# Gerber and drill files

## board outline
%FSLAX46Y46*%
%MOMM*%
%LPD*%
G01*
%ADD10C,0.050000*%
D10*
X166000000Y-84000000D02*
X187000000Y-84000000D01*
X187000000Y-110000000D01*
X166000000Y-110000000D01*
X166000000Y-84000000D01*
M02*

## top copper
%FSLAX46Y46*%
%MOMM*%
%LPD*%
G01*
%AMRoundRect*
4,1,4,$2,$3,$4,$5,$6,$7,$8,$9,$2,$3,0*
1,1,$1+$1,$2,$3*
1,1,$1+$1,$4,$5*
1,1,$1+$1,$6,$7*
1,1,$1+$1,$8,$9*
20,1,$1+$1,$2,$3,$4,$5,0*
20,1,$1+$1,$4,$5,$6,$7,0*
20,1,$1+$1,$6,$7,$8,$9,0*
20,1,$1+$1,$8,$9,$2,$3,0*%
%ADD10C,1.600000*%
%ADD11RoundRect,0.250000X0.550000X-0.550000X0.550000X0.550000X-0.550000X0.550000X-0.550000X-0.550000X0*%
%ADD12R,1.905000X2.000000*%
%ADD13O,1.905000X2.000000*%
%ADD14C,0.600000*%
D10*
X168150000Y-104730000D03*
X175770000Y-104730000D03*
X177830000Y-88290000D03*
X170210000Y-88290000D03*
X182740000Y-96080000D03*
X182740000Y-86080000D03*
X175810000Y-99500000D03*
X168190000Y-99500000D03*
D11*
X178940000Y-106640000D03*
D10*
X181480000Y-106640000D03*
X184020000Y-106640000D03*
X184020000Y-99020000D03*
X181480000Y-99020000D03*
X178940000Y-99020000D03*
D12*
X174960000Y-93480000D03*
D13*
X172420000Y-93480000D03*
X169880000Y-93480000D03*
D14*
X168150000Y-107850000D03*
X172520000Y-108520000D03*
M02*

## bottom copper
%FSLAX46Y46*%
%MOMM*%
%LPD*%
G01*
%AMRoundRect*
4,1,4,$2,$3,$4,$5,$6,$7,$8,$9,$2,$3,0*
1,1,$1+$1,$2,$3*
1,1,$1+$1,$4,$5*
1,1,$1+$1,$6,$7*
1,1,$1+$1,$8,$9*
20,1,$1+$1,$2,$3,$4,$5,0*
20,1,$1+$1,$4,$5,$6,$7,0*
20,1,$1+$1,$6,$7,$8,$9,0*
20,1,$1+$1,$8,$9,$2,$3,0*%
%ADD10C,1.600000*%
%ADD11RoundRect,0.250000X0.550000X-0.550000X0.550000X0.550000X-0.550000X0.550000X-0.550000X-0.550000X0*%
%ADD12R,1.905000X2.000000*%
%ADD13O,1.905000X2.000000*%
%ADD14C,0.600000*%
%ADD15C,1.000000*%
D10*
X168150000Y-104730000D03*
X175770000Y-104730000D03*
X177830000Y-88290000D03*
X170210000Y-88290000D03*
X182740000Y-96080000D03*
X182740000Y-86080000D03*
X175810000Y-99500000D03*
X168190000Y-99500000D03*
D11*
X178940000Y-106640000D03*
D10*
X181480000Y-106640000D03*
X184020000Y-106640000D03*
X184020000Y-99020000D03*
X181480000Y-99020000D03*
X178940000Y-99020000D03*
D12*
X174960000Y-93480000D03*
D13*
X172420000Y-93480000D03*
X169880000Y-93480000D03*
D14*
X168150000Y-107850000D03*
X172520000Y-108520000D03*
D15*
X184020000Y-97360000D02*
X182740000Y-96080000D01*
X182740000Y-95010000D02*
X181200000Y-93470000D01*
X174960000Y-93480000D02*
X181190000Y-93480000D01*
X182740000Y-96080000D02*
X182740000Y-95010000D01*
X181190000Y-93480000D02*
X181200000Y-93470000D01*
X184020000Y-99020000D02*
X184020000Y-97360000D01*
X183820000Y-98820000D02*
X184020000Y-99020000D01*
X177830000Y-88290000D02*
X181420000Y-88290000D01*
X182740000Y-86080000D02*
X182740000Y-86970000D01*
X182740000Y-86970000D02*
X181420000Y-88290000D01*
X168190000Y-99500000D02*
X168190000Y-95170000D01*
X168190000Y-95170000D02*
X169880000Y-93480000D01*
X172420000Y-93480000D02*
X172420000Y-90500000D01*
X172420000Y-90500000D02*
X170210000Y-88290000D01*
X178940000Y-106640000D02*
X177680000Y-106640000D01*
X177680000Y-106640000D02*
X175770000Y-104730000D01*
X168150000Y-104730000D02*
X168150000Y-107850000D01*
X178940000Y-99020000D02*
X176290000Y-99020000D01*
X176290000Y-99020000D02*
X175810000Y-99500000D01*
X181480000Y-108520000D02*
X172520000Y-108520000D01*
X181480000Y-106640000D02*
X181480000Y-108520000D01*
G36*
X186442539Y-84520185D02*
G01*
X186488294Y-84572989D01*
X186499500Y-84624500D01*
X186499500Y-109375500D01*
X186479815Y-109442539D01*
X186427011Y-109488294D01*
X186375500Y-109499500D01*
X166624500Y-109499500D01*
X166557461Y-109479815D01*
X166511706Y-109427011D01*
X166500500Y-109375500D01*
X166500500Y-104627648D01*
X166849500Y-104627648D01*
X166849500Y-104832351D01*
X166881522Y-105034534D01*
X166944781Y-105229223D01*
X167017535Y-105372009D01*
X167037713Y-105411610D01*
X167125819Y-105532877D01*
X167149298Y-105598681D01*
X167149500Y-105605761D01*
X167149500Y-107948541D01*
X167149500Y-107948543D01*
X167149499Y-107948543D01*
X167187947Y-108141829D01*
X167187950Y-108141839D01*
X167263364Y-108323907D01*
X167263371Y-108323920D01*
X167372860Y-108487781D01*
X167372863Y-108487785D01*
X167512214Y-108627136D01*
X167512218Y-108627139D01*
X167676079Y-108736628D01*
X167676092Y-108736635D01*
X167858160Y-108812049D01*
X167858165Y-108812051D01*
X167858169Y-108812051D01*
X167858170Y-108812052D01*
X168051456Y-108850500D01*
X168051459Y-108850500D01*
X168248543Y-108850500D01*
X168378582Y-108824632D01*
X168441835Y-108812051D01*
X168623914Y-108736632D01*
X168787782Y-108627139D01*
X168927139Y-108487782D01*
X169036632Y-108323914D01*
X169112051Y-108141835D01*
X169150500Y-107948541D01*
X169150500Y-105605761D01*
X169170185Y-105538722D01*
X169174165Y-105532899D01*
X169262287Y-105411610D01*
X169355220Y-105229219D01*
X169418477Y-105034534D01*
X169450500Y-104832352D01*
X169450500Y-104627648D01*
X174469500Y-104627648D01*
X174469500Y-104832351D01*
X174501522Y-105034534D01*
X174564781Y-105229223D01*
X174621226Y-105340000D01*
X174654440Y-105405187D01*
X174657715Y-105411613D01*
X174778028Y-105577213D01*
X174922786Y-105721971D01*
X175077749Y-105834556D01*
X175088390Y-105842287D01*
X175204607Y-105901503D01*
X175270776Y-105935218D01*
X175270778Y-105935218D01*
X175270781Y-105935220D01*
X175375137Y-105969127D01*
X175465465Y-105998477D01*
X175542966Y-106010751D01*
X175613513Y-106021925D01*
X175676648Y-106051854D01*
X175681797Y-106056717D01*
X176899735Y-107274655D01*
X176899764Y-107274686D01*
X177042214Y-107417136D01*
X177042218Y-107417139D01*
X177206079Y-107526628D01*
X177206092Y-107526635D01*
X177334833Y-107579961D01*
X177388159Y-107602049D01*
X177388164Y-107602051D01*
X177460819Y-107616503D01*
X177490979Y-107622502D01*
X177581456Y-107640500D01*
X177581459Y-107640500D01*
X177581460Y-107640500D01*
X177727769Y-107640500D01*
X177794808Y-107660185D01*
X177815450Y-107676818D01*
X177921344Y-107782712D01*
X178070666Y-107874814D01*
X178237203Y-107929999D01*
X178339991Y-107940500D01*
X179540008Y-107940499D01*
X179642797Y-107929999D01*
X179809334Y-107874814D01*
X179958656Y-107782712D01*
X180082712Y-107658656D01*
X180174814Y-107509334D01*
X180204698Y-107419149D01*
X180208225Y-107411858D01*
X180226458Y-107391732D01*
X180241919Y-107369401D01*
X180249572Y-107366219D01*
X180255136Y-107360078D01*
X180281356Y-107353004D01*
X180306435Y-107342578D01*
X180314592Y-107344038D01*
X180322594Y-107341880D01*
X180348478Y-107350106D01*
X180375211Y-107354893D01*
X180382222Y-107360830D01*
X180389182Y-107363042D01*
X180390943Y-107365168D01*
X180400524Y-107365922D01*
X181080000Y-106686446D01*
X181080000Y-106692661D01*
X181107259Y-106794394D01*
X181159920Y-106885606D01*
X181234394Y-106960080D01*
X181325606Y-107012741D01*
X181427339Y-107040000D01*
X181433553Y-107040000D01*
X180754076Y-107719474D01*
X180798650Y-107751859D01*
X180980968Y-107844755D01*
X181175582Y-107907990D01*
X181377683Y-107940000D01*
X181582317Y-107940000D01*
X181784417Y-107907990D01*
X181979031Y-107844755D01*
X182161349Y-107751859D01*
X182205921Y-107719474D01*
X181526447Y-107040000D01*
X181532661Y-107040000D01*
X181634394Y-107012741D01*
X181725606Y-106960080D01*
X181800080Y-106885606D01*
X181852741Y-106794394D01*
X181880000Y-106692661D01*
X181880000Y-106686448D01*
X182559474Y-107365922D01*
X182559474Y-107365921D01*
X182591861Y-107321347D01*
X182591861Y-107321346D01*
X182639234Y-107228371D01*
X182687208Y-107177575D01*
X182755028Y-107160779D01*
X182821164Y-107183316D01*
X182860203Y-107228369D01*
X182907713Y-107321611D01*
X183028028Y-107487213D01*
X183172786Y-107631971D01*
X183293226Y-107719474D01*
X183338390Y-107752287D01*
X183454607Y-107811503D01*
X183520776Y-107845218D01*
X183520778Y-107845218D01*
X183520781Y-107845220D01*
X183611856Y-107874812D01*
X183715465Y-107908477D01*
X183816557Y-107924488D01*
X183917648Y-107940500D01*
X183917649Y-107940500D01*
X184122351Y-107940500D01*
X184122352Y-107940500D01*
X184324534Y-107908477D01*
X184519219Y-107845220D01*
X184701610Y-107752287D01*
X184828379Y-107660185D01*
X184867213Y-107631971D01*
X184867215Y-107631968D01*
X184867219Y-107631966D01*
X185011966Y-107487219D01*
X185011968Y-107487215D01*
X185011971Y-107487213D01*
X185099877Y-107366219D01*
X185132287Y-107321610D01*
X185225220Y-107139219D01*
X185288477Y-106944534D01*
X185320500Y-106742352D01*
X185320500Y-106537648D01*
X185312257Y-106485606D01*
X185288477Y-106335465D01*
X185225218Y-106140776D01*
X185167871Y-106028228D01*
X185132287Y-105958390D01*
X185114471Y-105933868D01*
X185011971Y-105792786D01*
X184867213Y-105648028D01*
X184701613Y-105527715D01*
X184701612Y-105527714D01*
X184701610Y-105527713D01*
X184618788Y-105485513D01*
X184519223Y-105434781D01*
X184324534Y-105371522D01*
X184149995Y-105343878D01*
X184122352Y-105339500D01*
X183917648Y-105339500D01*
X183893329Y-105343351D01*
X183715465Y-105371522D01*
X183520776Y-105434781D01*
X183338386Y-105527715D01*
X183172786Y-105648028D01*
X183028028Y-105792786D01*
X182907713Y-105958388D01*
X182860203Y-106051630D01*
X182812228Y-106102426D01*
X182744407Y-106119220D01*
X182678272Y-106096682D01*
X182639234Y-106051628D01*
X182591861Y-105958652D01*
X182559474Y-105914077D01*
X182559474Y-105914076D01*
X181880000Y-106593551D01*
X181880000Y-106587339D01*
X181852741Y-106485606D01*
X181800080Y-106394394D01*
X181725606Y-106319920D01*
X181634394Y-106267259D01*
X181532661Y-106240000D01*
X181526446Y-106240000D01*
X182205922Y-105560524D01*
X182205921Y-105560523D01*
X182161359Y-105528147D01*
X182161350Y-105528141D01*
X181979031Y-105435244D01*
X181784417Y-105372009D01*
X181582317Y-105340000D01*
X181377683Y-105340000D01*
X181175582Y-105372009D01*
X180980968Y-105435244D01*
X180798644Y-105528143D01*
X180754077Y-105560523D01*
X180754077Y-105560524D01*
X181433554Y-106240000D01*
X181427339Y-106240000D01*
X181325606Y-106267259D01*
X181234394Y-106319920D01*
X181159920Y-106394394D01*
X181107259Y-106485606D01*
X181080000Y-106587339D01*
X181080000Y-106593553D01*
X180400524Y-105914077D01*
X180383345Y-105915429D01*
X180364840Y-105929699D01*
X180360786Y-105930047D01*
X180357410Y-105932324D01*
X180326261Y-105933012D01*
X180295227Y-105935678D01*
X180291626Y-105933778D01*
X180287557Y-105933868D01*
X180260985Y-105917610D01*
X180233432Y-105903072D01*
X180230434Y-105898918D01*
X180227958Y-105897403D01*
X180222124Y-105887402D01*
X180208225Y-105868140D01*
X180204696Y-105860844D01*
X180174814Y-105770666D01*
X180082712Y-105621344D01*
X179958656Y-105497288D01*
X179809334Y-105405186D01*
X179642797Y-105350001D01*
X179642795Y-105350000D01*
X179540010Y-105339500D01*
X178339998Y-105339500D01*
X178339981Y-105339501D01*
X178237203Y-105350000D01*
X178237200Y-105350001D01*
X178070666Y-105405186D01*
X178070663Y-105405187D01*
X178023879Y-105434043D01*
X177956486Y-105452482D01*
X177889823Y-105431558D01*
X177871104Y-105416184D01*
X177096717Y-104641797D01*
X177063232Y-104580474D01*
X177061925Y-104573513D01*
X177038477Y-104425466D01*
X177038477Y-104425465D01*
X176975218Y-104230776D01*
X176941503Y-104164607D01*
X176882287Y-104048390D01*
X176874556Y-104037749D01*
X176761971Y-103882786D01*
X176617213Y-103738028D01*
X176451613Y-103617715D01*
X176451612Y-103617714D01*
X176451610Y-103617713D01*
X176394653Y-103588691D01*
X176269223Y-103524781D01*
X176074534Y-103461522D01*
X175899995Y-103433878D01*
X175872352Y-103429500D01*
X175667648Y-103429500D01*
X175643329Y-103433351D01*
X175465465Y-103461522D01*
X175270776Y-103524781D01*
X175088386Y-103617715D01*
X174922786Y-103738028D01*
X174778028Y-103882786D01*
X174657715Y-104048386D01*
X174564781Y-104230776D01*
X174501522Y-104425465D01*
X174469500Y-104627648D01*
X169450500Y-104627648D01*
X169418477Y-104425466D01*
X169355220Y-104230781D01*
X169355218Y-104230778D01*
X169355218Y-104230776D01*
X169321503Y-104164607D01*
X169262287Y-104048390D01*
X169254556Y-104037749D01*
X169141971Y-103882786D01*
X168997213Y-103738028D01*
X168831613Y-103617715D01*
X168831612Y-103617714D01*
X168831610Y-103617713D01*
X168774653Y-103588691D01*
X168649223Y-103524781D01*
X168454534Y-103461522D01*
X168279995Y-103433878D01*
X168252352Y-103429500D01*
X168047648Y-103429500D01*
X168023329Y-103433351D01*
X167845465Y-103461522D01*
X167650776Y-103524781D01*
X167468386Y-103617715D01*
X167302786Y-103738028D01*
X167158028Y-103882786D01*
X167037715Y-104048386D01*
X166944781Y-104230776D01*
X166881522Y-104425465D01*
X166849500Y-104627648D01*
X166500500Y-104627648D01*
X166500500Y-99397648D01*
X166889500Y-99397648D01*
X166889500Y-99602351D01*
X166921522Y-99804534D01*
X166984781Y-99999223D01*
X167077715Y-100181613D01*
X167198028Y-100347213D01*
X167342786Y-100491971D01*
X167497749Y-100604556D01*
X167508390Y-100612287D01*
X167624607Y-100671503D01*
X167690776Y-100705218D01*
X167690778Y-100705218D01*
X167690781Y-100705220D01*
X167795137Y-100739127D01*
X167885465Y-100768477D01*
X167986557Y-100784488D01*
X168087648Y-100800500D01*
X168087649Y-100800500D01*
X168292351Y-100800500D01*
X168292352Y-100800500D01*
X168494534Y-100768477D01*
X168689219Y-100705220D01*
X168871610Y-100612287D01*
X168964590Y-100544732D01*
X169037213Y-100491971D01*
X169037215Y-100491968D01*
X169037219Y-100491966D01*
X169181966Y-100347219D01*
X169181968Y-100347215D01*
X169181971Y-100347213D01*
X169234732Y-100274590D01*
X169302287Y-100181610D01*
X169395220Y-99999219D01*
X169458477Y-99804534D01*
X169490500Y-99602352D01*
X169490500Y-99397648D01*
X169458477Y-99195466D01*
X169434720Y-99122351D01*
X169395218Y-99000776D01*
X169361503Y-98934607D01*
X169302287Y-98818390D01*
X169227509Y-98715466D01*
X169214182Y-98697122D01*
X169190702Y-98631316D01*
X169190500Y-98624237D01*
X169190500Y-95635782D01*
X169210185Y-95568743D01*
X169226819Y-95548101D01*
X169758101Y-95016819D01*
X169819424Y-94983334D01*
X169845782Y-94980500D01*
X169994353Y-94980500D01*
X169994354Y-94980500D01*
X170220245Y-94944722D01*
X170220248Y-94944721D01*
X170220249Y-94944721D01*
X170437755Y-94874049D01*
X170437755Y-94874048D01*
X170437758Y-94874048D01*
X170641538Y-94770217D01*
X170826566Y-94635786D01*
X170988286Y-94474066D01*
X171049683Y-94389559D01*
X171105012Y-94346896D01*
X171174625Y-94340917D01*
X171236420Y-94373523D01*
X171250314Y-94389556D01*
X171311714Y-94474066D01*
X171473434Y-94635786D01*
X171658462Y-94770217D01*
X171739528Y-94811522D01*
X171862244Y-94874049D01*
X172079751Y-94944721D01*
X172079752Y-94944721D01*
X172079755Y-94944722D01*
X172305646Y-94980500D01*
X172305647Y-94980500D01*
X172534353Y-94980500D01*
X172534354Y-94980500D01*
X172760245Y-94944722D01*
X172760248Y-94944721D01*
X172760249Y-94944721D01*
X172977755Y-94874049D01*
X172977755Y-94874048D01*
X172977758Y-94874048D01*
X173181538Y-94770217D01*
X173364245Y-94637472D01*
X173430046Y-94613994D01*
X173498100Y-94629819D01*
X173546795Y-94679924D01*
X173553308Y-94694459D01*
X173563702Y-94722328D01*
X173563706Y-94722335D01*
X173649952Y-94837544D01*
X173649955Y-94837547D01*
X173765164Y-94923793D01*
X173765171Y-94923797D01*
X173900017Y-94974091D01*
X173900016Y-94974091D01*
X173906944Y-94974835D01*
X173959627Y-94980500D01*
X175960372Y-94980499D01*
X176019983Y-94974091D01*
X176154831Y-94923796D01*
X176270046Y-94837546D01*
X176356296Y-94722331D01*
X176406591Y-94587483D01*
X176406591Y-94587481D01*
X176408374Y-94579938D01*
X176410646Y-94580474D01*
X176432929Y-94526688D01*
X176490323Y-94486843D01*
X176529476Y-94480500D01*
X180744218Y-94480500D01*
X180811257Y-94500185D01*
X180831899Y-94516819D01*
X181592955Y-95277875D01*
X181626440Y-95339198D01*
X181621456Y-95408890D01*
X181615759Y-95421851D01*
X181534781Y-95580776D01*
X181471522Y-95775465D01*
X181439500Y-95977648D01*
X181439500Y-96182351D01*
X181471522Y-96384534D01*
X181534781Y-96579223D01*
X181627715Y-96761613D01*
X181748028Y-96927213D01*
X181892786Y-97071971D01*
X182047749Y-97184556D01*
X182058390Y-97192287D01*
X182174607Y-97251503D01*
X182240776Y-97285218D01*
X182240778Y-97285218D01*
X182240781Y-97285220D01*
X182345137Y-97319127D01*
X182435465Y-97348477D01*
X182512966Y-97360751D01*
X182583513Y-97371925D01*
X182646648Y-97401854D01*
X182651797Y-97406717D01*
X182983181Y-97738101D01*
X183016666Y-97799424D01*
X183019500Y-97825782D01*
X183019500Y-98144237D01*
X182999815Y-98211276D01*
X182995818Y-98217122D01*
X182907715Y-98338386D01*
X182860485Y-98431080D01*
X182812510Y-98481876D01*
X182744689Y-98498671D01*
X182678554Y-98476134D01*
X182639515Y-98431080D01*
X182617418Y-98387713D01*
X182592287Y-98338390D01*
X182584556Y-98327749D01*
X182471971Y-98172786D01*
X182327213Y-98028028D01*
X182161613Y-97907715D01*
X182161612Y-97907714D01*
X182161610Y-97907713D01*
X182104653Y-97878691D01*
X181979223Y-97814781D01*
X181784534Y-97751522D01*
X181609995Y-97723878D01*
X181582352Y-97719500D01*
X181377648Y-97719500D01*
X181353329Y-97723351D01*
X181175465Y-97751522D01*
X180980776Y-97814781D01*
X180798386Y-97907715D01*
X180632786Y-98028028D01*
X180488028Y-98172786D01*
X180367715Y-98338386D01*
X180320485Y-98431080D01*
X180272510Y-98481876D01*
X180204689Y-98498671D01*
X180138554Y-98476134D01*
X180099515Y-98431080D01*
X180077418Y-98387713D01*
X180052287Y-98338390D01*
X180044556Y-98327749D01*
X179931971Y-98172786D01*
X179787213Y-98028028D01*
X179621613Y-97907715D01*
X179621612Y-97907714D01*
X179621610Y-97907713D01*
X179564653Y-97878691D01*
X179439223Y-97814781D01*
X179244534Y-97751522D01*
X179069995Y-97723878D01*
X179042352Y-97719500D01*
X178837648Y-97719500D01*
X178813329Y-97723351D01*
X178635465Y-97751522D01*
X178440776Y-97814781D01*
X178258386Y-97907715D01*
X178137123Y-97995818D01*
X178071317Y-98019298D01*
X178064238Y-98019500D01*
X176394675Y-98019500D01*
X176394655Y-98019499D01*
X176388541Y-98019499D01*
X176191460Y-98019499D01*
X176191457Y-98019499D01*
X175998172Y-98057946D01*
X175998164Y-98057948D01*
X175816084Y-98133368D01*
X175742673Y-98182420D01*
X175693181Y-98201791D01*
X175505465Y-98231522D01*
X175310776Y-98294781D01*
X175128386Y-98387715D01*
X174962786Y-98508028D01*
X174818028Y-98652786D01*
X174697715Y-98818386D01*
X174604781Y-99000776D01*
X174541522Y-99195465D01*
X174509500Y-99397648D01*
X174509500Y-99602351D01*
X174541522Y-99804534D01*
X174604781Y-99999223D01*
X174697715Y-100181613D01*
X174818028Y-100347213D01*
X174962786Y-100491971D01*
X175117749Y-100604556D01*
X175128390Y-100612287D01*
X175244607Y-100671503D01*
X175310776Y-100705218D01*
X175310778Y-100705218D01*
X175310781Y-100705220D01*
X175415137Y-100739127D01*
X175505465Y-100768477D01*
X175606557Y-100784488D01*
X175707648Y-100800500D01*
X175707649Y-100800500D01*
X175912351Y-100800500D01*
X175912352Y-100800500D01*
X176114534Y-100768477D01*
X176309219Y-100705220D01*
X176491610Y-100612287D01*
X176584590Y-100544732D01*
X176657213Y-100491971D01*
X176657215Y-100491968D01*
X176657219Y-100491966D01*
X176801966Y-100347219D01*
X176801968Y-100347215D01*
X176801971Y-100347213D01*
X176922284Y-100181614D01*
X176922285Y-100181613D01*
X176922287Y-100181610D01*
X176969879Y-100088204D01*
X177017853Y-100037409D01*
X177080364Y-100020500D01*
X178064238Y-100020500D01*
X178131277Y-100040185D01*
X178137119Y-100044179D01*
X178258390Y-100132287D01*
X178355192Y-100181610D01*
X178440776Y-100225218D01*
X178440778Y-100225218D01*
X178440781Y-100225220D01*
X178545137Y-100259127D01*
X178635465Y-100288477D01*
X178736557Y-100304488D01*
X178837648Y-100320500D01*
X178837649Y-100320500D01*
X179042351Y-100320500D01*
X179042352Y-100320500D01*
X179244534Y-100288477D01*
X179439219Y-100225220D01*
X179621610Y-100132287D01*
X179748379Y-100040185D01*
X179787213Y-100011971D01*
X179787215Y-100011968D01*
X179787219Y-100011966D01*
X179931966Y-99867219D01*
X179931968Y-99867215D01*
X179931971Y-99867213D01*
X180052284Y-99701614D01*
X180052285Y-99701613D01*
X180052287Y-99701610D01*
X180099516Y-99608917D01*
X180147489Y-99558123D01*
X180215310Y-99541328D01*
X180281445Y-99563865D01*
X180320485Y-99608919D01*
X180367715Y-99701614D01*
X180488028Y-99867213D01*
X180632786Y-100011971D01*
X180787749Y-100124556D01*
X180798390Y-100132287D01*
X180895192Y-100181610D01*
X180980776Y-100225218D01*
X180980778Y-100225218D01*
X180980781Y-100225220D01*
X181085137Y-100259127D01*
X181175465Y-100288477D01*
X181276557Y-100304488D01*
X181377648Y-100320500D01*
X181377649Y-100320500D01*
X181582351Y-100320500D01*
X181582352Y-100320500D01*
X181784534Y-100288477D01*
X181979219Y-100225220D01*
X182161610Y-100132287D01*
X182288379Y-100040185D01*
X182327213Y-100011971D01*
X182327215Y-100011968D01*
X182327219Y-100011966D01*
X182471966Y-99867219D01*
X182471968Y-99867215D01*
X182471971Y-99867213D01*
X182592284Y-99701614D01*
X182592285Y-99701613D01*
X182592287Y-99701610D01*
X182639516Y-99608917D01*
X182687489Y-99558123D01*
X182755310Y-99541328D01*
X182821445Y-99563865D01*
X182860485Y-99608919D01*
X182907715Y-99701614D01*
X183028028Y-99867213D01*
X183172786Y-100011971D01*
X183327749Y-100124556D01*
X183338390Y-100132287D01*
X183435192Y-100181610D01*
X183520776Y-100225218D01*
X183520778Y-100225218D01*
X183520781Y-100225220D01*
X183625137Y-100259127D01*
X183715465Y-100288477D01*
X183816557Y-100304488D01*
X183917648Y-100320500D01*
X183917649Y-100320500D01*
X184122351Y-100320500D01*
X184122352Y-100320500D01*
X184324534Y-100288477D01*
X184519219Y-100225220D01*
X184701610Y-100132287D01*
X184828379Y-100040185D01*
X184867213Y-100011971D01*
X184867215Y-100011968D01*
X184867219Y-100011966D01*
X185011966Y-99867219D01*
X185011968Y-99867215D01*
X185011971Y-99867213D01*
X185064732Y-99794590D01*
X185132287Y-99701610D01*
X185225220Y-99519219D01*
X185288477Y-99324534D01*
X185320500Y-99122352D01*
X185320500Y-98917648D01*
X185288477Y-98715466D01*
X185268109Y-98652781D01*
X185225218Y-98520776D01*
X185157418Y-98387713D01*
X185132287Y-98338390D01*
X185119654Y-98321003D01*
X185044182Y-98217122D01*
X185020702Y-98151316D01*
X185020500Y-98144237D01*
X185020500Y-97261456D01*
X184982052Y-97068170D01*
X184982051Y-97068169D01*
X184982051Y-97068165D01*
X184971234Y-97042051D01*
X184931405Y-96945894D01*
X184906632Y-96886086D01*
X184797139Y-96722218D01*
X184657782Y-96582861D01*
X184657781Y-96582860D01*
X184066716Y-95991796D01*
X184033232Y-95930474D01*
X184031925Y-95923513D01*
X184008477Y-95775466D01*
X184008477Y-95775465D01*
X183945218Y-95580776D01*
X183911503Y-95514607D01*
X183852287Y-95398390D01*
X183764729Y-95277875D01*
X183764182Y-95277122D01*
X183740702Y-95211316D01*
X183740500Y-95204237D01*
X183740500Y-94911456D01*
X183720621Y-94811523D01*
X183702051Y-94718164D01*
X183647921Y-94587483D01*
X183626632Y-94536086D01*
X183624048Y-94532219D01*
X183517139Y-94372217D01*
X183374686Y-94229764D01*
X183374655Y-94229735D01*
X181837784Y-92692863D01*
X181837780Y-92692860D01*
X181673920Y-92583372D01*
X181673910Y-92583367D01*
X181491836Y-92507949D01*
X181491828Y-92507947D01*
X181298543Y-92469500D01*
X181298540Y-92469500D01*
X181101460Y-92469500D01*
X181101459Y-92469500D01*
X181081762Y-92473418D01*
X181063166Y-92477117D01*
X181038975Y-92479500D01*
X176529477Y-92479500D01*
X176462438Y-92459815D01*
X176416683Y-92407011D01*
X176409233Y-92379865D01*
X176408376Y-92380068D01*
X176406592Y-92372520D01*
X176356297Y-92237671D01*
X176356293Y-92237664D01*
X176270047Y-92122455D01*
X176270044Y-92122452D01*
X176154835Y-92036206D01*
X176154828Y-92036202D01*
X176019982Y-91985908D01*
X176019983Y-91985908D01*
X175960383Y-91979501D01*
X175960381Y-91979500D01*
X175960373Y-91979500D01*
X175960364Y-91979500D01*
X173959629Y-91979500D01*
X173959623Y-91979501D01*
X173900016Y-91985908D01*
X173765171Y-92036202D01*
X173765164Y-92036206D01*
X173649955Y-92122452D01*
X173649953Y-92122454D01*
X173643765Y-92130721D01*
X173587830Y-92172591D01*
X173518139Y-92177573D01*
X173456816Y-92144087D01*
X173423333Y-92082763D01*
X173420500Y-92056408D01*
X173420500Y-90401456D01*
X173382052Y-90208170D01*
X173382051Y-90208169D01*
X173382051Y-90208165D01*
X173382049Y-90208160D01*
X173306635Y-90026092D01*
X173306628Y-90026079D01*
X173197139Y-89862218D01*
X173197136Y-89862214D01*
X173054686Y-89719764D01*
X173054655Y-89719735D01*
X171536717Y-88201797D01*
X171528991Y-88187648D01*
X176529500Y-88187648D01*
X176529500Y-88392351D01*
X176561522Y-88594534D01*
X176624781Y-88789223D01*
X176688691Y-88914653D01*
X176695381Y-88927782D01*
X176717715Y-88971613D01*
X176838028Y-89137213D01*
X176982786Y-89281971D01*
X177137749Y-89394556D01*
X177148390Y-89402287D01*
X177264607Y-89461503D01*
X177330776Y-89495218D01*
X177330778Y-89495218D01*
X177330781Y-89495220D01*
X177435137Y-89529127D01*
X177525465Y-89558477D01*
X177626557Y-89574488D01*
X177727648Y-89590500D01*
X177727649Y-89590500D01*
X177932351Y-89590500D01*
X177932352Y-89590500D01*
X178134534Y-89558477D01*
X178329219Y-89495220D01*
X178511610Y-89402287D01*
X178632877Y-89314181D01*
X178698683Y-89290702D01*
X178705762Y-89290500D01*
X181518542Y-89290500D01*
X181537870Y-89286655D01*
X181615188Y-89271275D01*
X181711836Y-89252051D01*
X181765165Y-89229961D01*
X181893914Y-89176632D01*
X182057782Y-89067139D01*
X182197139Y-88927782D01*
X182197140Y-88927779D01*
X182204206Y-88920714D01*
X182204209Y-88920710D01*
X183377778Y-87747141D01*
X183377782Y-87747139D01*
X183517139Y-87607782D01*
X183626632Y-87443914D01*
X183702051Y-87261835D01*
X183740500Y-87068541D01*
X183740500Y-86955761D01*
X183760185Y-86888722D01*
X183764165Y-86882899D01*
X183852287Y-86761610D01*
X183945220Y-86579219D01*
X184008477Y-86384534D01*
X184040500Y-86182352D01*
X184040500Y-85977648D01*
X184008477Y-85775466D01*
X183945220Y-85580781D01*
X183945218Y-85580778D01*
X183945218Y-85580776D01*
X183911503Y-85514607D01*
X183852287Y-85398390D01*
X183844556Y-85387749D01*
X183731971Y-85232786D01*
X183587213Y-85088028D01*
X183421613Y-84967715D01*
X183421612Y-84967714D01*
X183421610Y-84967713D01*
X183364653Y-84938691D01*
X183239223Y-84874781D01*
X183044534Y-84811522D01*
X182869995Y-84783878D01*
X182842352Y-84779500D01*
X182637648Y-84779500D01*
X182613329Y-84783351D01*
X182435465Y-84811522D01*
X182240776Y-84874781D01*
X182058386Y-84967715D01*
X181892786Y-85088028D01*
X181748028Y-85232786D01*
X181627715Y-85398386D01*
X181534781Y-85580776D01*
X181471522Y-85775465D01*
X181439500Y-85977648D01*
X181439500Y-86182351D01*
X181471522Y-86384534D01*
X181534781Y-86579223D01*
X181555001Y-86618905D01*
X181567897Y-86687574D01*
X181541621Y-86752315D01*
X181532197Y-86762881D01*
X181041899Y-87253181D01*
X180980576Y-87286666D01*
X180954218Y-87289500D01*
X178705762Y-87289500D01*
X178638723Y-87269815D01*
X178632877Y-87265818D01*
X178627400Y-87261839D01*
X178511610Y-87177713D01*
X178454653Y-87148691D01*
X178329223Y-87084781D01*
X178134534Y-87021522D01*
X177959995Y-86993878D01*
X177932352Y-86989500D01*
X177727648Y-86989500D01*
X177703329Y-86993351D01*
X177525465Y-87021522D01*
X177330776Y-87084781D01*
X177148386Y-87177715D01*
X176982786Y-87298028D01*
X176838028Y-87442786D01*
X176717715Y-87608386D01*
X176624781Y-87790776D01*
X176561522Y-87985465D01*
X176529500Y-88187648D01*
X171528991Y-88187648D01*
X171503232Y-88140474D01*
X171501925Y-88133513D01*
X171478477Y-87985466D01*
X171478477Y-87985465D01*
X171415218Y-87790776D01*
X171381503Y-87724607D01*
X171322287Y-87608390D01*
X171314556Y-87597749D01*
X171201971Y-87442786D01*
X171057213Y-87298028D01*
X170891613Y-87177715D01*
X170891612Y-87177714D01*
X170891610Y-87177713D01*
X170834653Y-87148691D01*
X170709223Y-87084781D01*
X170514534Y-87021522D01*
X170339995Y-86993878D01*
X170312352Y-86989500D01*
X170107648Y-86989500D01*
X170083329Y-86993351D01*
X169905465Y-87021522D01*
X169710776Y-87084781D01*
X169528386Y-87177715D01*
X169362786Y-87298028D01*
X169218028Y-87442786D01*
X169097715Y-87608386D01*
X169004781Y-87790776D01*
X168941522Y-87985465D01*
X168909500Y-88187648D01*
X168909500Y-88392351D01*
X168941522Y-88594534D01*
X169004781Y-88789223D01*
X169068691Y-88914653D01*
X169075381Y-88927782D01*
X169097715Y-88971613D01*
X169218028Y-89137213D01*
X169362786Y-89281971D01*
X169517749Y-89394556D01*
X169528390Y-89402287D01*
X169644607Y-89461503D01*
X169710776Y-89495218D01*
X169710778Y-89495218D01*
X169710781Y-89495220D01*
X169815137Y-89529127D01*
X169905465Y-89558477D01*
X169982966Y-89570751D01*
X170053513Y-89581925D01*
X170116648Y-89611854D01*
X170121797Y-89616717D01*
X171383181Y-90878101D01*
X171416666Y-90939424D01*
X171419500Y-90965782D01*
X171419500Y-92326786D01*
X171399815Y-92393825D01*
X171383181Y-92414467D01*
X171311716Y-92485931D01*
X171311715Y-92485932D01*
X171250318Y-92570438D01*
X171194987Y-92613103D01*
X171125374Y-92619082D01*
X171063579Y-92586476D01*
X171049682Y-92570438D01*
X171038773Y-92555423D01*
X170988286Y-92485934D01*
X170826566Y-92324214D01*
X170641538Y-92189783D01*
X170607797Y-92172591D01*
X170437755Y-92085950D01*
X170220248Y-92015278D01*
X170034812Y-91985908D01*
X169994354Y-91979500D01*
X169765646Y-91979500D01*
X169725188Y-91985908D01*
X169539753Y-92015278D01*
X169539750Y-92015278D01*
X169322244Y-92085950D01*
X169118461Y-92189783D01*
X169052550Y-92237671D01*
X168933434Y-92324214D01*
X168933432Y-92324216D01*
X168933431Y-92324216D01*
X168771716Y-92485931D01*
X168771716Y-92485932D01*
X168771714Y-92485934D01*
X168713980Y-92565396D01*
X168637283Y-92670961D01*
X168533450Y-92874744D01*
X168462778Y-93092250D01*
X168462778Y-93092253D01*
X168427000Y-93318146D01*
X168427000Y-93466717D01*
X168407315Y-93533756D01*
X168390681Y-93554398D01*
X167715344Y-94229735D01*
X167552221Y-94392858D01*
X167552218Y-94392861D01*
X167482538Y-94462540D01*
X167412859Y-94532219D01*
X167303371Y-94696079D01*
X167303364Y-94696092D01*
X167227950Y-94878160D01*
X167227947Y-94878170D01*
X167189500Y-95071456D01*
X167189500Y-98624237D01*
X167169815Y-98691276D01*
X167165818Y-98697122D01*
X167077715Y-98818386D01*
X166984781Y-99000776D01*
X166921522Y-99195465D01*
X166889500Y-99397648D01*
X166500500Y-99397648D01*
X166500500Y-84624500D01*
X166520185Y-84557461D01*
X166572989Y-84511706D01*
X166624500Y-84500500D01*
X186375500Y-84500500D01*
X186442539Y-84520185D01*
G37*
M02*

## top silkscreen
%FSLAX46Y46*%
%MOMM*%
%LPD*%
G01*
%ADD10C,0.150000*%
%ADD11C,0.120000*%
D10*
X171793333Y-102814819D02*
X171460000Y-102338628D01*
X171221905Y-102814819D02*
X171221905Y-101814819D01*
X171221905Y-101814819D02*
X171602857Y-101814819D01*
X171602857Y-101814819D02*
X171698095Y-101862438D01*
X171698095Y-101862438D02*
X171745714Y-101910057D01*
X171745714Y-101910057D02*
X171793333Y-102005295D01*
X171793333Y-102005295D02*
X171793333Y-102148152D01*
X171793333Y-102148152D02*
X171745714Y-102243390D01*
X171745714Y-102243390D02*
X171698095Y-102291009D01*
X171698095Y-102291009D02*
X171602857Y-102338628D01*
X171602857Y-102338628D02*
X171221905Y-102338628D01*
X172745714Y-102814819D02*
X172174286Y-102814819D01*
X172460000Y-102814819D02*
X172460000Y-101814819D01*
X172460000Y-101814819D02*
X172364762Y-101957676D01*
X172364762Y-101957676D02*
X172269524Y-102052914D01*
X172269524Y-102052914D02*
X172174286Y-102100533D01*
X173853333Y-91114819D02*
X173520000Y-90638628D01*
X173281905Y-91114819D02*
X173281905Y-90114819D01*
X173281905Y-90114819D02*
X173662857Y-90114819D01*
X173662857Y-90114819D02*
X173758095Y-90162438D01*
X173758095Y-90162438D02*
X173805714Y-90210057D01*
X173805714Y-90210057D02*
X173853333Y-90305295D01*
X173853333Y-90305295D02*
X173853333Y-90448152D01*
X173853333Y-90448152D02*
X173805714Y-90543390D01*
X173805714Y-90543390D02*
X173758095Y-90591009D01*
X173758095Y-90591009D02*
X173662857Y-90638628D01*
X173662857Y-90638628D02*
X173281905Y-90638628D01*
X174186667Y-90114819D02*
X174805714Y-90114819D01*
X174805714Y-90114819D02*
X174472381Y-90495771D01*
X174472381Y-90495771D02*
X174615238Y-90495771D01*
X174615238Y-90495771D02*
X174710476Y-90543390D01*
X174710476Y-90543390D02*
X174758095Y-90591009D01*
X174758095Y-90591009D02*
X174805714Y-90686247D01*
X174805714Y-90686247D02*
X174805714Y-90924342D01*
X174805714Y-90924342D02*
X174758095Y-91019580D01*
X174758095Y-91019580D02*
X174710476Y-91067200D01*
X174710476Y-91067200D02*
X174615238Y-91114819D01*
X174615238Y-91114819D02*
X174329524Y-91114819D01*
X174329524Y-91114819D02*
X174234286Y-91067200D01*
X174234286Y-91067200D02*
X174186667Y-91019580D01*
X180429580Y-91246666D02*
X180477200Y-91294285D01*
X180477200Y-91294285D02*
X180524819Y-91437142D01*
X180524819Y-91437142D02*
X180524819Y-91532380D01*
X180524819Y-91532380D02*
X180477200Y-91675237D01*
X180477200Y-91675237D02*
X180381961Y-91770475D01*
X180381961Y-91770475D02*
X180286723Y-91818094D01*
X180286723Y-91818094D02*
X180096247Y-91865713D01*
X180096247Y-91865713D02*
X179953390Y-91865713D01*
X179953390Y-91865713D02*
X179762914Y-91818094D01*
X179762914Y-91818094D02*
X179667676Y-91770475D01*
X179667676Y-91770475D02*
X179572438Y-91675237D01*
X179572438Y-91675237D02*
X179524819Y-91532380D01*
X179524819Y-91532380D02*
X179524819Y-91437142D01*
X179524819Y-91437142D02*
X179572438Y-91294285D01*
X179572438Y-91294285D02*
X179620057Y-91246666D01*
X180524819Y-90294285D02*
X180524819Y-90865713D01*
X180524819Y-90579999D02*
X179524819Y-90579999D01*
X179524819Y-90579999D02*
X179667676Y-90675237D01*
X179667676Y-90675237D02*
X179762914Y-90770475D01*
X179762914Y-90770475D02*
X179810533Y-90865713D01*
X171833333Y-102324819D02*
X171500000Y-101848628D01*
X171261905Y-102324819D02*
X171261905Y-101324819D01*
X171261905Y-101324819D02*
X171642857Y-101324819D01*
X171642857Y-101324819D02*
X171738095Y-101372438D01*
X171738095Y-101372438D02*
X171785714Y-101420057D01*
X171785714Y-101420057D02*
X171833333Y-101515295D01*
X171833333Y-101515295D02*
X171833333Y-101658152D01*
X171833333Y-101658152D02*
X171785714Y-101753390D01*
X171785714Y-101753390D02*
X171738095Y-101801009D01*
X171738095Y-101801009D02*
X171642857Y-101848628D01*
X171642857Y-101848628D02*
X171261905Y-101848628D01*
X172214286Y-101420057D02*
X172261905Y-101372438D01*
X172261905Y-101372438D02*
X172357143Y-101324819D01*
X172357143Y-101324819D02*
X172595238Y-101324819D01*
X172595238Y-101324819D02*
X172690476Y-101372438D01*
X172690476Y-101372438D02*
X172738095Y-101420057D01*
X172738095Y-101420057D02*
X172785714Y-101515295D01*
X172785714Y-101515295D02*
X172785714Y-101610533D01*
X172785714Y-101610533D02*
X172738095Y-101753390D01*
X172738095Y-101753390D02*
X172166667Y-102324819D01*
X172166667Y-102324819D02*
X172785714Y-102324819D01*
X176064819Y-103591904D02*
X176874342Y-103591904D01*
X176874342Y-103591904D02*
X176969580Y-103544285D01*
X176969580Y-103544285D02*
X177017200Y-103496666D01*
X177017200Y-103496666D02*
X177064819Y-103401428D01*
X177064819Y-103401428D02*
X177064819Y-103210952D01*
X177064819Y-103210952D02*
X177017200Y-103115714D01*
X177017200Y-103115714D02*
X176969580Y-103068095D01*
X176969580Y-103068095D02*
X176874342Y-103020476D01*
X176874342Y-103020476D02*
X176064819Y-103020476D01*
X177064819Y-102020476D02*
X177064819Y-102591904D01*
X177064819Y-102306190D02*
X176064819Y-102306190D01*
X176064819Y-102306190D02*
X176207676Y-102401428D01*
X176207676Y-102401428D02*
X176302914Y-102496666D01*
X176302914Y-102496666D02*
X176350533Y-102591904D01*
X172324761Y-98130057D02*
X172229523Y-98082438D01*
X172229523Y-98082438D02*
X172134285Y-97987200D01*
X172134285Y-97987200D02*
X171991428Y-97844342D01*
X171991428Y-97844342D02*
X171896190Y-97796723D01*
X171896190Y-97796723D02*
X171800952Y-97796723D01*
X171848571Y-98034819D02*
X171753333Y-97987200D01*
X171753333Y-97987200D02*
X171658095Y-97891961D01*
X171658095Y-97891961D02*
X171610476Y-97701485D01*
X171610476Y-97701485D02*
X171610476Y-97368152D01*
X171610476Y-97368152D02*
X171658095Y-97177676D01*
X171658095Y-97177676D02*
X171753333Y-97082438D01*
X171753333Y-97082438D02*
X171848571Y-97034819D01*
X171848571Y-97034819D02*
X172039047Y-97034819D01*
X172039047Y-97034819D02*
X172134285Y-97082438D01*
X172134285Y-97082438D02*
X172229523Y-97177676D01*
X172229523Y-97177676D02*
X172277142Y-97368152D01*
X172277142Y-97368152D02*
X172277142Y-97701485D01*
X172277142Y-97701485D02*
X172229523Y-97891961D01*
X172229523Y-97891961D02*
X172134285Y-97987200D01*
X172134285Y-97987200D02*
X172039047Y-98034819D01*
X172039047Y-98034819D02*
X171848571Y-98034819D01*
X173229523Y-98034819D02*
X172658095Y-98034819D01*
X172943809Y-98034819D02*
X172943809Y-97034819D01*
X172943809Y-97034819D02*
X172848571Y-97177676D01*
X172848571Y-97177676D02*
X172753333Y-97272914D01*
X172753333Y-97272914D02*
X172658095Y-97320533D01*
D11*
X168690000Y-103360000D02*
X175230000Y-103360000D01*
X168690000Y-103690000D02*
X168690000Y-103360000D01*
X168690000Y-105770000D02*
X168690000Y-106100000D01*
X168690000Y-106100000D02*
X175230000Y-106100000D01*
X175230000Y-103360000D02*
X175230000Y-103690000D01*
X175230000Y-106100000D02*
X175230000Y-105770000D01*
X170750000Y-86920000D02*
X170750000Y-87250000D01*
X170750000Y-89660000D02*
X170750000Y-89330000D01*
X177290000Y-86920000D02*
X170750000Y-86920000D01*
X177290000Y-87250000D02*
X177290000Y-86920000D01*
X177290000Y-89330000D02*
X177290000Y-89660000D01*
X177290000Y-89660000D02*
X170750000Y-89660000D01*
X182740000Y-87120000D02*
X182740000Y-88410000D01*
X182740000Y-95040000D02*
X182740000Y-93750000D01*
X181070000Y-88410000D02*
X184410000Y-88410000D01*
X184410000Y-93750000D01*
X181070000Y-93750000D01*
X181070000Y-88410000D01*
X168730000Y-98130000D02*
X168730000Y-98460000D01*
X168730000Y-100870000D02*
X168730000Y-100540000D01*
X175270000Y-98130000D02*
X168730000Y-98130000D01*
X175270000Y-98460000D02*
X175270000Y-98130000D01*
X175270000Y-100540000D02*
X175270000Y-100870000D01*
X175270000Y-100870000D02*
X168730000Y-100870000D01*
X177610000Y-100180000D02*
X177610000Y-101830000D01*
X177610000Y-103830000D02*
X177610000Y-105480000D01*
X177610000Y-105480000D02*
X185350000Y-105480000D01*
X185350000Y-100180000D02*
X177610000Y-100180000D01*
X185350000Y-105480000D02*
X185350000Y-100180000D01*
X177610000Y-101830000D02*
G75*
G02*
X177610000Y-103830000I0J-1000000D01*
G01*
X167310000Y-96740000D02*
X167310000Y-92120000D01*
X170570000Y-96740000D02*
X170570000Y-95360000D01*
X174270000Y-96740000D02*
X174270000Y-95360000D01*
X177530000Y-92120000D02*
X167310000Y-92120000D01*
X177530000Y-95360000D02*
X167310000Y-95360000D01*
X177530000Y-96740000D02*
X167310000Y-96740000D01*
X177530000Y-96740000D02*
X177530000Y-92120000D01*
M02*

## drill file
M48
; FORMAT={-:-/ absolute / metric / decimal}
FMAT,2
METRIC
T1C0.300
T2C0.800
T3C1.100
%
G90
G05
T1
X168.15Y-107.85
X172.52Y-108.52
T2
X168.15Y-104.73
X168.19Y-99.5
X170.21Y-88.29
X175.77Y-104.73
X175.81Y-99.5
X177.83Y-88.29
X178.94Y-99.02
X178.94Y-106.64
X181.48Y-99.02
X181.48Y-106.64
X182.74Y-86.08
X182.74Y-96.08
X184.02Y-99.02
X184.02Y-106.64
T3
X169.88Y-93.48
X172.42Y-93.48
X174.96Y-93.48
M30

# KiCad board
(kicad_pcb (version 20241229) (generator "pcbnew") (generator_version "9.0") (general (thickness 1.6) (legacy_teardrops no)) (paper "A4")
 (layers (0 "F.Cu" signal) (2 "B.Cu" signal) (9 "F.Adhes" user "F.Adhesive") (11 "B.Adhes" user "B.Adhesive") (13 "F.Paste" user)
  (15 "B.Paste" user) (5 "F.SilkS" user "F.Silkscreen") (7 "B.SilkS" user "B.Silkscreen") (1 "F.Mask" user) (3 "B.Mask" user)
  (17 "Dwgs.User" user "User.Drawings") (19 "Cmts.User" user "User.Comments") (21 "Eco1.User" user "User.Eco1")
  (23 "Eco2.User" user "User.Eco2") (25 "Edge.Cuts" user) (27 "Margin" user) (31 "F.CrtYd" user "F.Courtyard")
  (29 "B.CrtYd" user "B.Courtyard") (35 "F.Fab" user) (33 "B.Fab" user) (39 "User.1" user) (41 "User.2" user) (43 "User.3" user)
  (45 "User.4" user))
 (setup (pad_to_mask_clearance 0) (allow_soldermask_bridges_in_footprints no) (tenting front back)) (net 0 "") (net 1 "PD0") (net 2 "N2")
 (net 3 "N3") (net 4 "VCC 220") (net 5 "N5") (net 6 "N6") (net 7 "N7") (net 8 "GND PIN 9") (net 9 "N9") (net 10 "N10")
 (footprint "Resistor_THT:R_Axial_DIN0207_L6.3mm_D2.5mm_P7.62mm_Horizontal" (layer "F.Cu") (at 168.15 104.73)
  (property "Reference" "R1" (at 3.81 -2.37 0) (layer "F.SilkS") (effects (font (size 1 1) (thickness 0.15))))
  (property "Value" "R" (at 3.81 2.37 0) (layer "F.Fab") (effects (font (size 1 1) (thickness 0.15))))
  (fp_line (start 0.54 -1.37) (end 7.08 -1.37) (stroke (width 0.12) (type solid)) (layer "F.SilkS"))
  (fp_line (start 0.54 -1.04) (end 0.54 -1.37) (stroke (width 0.12) (type solid)) (layer "F.SilkS"))
  (fp_line (start 0.54 1.04) (end 0.54 1.37) (stroke (width 0.12) (type solid)) (layer "F.SilkS"))
  (fp_line (start 0.54 1.37) (end 7.08 1.37) (stroke (width 0.12) (type solid)) (layer "F.SilkS"))
  (fp_line (start 7.08 -1.37) (end 7.08 -1.04) (stroke (width 0.12) (type solid)) (layer "F.SilkS"))
  (fp_line (start 7.08 1.37) (end 7.08 1.04) (stroke (width 0.12) (type solid)) (layer "F.SilkS"))
  (pad "1" thru_hole circle (at 0 0) (size 1.6 1.6) (drill 0.8) (layers "*.Cu" "*.Mask") (remove_unused_layers no) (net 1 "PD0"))
  (pad "2" thru_hole circle (at 7.62 0) (size 1.6 1.6) (drill 0.8) (layers "*.Cu" "*.Mask") (remove_unused_layers no) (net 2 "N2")))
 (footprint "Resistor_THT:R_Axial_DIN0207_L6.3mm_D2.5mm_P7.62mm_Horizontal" (layer "F.Cu") (at 177.83 88.29 180)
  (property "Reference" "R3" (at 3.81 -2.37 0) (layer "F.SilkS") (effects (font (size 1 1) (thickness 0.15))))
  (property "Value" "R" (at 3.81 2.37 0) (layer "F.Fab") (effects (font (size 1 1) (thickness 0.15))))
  (fp_line (start 7.08 1.37) (end 7.08 1.04) (stroke (width 0.12) (type solid)) (layer "F.SilkS"))
  (fp_line (start 7.08 -1.37) (end 7.08 -1.04) (stroke (width 0.12) (type solid)) (layer "F.SilkS"))
  (fp_line (start 0.54 1.37) (end 7.08 1.37) (stroke (width 0.12) (type solid)) (layer "F.SilkS"))
  (fp_line (start 0.54 1.04) (end 0.54 1.37) (stroke (width 0.12) (type solid)) (layer "F.SilkS"))
  (fp_line (start 0.54 -1.04) (end 0.54 -1.37) (stroke (width 0.12) (type solid)) (layer "F.SilkS"))
  (fp_line (start 0.54 -1.37) (end 7.08 -1.37) (stroke (width 0.12) (type solid)) (layer "F.SilkS"))
  (pad "1" thru_hole circle (at 0 0 180) (size 1.6 1.6) (drill 0.8) (layers "*.Cu" "*.Mask") (remove_unused_layers no) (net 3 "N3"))
  (pad "2" thru_hole circle (at 7.62 0 180) (size 1.6 1.6) (drill 0.8) (layers "*.Cu" "*.Mask") (remove_unused_layers no) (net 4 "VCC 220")))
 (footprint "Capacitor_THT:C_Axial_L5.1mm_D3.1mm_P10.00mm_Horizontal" (layer "F.Cu") (at 182.74 96.08 90)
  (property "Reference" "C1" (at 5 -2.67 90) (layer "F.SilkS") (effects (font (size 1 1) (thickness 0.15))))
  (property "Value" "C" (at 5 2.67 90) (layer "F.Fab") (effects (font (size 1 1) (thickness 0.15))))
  (fp_line (start 8.96 0) (end 7.67 0) (stroke (width 0.12) (type solid)) (layer "F.SilkS"))
  (fp_line (start 1.04 0) (end 2.33 0) (stroke (width 0.12) (type solid)) (layer "F.SilkS"))
  (fp_rect (start 2.33 -1.67) (end 7.67 1.67) (stroke (width 0.12) (type solid)) (fill no) (layer "F.SilkS"))
  (pad "1" thru_hole circle (at 0 0 90) (size 1.6 1.6) (drill 0.8) (layers "*.Cu" "*.Mask") (remove_unused_layers no) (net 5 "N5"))
  (pad "2" thru_hole circle (at 10 0 90) (size 1.6 1.6) (drill 0.8) (layers "*.Cu" "*.Mask") (remove_unused_layers no) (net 3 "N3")))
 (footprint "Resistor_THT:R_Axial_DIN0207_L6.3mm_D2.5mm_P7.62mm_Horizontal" (layer "F.Cu") (at 175.81 99.5 180)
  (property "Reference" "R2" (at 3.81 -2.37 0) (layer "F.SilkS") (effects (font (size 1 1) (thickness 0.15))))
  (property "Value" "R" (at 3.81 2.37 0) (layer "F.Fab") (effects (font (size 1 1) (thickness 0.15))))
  (fp_line (start 7.08 1.37) (end 7.08 1.04) (stroke (width 0.12) (type solid)) (layer "F.SilkS"))
  (fp_line (start 7.08 -1.37) (end 7.08 -1.04) (stroke (width 0.12) (type solid)) (layer "F.SilkS"))
  (fp_line (start 0.54 1.37) (end 7.08 1.37) (stroke (width 0.12) (type solid)) (layer "F.SilkS"))
  (fp_line (start 0.54 1.04) (end 0.54 1.37) (stroke (width 0.12) (type solid)) (layer "F.SilkS"))
  (fp_line (start 0.54 -1.04) (end 0.54 -1.37) (stroke (width 0.12) (type solid)) (layer "F.SilkS"))
  (fp_line (start 0.54 -1.37) (end 7.08 -1.37) (stroke (width 0.12) (type solid)) (layer "F.SilkS"))
  (pad "1" thru_hole circle (at 0 0 180) (size 1.6 1.6) (drill 0.8) (layers "*.Cu" "*.Mask") (remove_unused_layers no) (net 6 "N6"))
  (pad "2" thru_hole circle (at 7.62 0 180) (size 1.6 1.6) (drill 0.8) (layers "*.Cu" "*.Mask") (remove_unused_layers no) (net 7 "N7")))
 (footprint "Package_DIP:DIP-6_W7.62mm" (layer "F.Cu") (at 178.94 106.64 90)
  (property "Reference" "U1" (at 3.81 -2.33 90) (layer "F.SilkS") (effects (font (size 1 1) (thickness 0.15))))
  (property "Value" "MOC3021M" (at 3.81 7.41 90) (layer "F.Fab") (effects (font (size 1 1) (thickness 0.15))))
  (fp_line (start 6.46 -1.33) (end 4.81 -1.33) (stroke (width 0.12) (type solid)) (layer "F.SilkS"))
  (fp_line (start 2.81 -1.33) (end 1.16 -1.33) (stroke (width 0.12) (type solid)) (layer "F.SilkS"))
  (fp_line (start 1.16 -1.33) (end 1.16 6.41) (stroke (width 0.12) (type solid)) (layer "F.SilkS"))
  (fp_line (start 6.46 6.41) (end 6.46 -1.33) (stroke (width 0.12) (type solid)) (layer "F.SilkS"))
  (fp_line (start 1.16 6.41) (end 6.46 6.41) (stroke (width 0.12) (type solid)) (layer "F.SilkS"))
  (fp_arc (start 4.81 -1.33) (mid 3.81 -0.33) (end 2.81 -1.33) (stroke (width 0.12) (type solid)) (layer "F.SilkS"))
  (pad "1" thru_hole roundrect (at 0 0 90) (size 1.6 1.6) (drill 0.8) (layers "*.Cu" "*.Mask") (remove_unused_layers no)
   (roundrect_rratio 0.15625) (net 2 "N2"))
  (pad "2" thru_hole circle (at 0 2.54 90) (size 1.6 1.6) (drill 0.8) (layers "*.Cu" "*.Mask") (remove_unused_layers no) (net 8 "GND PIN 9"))
  (pad "3" thru_hole circle (at 0 5.08 90) (size 1.6 1.6) (drill 0.8) (layers "*.Cu" "*.Mask") (remove_unused_layers no) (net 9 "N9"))
  (pad "4" thru_hole circle (at 7.62 5.08 90) (size 1.6 1.6) (drill 0.8) (layers "*.Cu" "*.Mask") (remove_unused_layers no) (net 5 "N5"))
  (pad "5" thru_hole circle (at 7.62 2.54 90) (size 1.6 1.6) (drill 0.8) (layers "*.Cu" "*.Mask") (remove_unused_layers no) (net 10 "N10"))
  (pad "6" thru_hole circle (at 7.62 0 90) (size 1.6 1.6) (drill 0.8) (layers "*.Cu" "*.Mask") (remove_unused_layers no) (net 6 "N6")))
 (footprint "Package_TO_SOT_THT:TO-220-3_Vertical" (layer "F.Cu") (at 174.96 93.48 180)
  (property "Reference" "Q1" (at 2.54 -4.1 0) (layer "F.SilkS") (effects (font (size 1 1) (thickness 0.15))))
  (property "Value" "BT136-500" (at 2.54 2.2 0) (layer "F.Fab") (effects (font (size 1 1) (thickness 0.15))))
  (fp_line (start 7.65 -3.26) (end 7.65 1.36) (stroke (width 0.12) (type solid)) (layer "F.SilkS"))
  (fp_line (start 4.39 -3.26) (end 4.39 -1.88) (stroke (width 0.12) (type solid)) (layer "F.SilkS"))
  (fp_line (start 0.69 -3.26) (end 0.69 -1.88) (stroke (width 0.12) (type solid)) (layer "F.SilkS"))
  (fp_line (start -2.57 1.36) (end 7.65 1.36) (stroke (width 0.12) (type solid)) (layer "F.SilkS"))
  (fp_line (start -2.57 -1.88) (end 7.65 -1.88) (stroke (width 0.12) (type solid)) (layer "F.SilkS"))
  (fp_line (start -2.57 -3.26) (end 7.65 -3.26) (stroke (width 0.12) (type solid)) (layer "F.SilkS"))
  (fp_line (start -2.57 -3.26) (end -2.57 1.36) (stroke (width 0.12) (type solid)) (layer "F.SilkS"))
  (pad "1" thru_hole rect (at 0 0 180) (size 1.905 2) (drill 1.1) (layers "*.Cu" "*.Mask") (remove_unused_layers no) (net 5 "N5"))
  (pad "2" thru_hole oval (at 2.54 0 180) (size 1.905 2) (drill 1.1) (layers "*.Cu" "*.Mask") (remove_unused_layers no) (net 4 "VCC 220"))
  (pad "3" thru_hole oval (at 5.08 0 180) (size 1.905 2) (drill 1.1) (layers "*.Cu" "*.Mask") (remove_unused_layers no) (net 7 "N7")))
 (gr_rect (start 166 84) (end 187 110) (stroke (width 0.05) (type default)) (fill no) (layer "Edge.Cuts"))
 (segment (start 184.02 97.36) (end 182.74 96.08) (width 1) (layer "B.Cu") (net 5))
 (segment (start 182.74 95.01) (end 181.2 93.47) (width 1) (layer "B.Cu") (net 5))
 (segment (start 174.96 93.48) (end 181.19 93.48) (width 1) (layer "B.Cu") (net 5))
 (segment (start 182.74 96.08) (end 182.74 95.01) (width 1) (layer "B.Cu") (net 5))
 (segment (start 181.19 93.48) (end 181.2 93.47) (width 1) (layer "B.Cu") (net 5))
 (segment (start 184.02 99.02) (end 184.02 97.36) (width 1) (layer "B.Cu") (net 5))
 (segment (start 183.82 98.82) (end 184.02 99.02) (width 1) (layer "B.Cu") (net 5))
 (segment (start 177.83 88.29) (end 181.42 88.29) (width 1) (layer "B.Cu") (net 3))
 (segment (start 182.74 86.08) (end 182.74 86.97) (width 1) (layer "B.Cu") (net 3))
 (segment (start 182.74 86.97) (end 181.42 88.29) (width 1) (layer "B.Cu") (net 3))
 (segment (start 168.19 99.5) (end 168.19 95.17) (width 1) (layer "B.Cu") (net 7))
 (segment (start 168.19 95.17) (end 169.88 93.48) (width 1) (layer "B.Cu") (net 7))
 (segment (start 172.42 93.48) (end 172.42 90.5) (width 1) (layer "B.Cu") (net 4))
 (segment (start 172.42 90.5) (end 170.21 88.29) (width 1) (layer "B.Cu") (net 4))
 (segment (start 178.94 106.64) (end 177.68 106.64) (width 1) (layer "B.Cu") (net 2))
 (segment (start 177.68 106.64) (end 175.77 104.73) (width 1) (layer "B.Cu") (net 2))
 (via (at 168.15 107.85) (size 0.6) (drill 0.3) (layers "F.Cu" "B.Cu") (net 1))
 (segment (start 168.15 104.73) (end 168.15 107.85) (width 1) (layer "B.Cu") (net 1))
 (segment (start 178.94 99.02) (end 176.29 99.02) (width 1) (layer "B.Cu") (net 6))
 (segment (start 176.29 99.02) (end 175.81 99.5) (width 1) (layer "B.Cu") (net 6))
 (via (at 172.52 108.52) (size 0.6) (drill 0.3) (layers "F.Cu" "B.Cu") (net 8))
 (segment (start 181.48 108.52) (end 172.52 108.52) (width 1) (layer "B.Cu") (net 8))
 (segment (start 181.48 106.64) (end 181.48 108.52) (width 1) (layer "B.Cu") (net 8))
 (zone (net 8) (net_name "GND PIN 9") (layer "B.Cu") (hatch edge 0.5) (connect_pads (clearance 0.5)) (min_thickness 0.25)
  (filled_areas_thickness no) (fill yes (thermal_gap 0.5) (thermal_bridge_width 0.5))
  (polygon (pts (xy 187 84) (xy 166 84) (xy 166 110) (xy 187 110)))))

